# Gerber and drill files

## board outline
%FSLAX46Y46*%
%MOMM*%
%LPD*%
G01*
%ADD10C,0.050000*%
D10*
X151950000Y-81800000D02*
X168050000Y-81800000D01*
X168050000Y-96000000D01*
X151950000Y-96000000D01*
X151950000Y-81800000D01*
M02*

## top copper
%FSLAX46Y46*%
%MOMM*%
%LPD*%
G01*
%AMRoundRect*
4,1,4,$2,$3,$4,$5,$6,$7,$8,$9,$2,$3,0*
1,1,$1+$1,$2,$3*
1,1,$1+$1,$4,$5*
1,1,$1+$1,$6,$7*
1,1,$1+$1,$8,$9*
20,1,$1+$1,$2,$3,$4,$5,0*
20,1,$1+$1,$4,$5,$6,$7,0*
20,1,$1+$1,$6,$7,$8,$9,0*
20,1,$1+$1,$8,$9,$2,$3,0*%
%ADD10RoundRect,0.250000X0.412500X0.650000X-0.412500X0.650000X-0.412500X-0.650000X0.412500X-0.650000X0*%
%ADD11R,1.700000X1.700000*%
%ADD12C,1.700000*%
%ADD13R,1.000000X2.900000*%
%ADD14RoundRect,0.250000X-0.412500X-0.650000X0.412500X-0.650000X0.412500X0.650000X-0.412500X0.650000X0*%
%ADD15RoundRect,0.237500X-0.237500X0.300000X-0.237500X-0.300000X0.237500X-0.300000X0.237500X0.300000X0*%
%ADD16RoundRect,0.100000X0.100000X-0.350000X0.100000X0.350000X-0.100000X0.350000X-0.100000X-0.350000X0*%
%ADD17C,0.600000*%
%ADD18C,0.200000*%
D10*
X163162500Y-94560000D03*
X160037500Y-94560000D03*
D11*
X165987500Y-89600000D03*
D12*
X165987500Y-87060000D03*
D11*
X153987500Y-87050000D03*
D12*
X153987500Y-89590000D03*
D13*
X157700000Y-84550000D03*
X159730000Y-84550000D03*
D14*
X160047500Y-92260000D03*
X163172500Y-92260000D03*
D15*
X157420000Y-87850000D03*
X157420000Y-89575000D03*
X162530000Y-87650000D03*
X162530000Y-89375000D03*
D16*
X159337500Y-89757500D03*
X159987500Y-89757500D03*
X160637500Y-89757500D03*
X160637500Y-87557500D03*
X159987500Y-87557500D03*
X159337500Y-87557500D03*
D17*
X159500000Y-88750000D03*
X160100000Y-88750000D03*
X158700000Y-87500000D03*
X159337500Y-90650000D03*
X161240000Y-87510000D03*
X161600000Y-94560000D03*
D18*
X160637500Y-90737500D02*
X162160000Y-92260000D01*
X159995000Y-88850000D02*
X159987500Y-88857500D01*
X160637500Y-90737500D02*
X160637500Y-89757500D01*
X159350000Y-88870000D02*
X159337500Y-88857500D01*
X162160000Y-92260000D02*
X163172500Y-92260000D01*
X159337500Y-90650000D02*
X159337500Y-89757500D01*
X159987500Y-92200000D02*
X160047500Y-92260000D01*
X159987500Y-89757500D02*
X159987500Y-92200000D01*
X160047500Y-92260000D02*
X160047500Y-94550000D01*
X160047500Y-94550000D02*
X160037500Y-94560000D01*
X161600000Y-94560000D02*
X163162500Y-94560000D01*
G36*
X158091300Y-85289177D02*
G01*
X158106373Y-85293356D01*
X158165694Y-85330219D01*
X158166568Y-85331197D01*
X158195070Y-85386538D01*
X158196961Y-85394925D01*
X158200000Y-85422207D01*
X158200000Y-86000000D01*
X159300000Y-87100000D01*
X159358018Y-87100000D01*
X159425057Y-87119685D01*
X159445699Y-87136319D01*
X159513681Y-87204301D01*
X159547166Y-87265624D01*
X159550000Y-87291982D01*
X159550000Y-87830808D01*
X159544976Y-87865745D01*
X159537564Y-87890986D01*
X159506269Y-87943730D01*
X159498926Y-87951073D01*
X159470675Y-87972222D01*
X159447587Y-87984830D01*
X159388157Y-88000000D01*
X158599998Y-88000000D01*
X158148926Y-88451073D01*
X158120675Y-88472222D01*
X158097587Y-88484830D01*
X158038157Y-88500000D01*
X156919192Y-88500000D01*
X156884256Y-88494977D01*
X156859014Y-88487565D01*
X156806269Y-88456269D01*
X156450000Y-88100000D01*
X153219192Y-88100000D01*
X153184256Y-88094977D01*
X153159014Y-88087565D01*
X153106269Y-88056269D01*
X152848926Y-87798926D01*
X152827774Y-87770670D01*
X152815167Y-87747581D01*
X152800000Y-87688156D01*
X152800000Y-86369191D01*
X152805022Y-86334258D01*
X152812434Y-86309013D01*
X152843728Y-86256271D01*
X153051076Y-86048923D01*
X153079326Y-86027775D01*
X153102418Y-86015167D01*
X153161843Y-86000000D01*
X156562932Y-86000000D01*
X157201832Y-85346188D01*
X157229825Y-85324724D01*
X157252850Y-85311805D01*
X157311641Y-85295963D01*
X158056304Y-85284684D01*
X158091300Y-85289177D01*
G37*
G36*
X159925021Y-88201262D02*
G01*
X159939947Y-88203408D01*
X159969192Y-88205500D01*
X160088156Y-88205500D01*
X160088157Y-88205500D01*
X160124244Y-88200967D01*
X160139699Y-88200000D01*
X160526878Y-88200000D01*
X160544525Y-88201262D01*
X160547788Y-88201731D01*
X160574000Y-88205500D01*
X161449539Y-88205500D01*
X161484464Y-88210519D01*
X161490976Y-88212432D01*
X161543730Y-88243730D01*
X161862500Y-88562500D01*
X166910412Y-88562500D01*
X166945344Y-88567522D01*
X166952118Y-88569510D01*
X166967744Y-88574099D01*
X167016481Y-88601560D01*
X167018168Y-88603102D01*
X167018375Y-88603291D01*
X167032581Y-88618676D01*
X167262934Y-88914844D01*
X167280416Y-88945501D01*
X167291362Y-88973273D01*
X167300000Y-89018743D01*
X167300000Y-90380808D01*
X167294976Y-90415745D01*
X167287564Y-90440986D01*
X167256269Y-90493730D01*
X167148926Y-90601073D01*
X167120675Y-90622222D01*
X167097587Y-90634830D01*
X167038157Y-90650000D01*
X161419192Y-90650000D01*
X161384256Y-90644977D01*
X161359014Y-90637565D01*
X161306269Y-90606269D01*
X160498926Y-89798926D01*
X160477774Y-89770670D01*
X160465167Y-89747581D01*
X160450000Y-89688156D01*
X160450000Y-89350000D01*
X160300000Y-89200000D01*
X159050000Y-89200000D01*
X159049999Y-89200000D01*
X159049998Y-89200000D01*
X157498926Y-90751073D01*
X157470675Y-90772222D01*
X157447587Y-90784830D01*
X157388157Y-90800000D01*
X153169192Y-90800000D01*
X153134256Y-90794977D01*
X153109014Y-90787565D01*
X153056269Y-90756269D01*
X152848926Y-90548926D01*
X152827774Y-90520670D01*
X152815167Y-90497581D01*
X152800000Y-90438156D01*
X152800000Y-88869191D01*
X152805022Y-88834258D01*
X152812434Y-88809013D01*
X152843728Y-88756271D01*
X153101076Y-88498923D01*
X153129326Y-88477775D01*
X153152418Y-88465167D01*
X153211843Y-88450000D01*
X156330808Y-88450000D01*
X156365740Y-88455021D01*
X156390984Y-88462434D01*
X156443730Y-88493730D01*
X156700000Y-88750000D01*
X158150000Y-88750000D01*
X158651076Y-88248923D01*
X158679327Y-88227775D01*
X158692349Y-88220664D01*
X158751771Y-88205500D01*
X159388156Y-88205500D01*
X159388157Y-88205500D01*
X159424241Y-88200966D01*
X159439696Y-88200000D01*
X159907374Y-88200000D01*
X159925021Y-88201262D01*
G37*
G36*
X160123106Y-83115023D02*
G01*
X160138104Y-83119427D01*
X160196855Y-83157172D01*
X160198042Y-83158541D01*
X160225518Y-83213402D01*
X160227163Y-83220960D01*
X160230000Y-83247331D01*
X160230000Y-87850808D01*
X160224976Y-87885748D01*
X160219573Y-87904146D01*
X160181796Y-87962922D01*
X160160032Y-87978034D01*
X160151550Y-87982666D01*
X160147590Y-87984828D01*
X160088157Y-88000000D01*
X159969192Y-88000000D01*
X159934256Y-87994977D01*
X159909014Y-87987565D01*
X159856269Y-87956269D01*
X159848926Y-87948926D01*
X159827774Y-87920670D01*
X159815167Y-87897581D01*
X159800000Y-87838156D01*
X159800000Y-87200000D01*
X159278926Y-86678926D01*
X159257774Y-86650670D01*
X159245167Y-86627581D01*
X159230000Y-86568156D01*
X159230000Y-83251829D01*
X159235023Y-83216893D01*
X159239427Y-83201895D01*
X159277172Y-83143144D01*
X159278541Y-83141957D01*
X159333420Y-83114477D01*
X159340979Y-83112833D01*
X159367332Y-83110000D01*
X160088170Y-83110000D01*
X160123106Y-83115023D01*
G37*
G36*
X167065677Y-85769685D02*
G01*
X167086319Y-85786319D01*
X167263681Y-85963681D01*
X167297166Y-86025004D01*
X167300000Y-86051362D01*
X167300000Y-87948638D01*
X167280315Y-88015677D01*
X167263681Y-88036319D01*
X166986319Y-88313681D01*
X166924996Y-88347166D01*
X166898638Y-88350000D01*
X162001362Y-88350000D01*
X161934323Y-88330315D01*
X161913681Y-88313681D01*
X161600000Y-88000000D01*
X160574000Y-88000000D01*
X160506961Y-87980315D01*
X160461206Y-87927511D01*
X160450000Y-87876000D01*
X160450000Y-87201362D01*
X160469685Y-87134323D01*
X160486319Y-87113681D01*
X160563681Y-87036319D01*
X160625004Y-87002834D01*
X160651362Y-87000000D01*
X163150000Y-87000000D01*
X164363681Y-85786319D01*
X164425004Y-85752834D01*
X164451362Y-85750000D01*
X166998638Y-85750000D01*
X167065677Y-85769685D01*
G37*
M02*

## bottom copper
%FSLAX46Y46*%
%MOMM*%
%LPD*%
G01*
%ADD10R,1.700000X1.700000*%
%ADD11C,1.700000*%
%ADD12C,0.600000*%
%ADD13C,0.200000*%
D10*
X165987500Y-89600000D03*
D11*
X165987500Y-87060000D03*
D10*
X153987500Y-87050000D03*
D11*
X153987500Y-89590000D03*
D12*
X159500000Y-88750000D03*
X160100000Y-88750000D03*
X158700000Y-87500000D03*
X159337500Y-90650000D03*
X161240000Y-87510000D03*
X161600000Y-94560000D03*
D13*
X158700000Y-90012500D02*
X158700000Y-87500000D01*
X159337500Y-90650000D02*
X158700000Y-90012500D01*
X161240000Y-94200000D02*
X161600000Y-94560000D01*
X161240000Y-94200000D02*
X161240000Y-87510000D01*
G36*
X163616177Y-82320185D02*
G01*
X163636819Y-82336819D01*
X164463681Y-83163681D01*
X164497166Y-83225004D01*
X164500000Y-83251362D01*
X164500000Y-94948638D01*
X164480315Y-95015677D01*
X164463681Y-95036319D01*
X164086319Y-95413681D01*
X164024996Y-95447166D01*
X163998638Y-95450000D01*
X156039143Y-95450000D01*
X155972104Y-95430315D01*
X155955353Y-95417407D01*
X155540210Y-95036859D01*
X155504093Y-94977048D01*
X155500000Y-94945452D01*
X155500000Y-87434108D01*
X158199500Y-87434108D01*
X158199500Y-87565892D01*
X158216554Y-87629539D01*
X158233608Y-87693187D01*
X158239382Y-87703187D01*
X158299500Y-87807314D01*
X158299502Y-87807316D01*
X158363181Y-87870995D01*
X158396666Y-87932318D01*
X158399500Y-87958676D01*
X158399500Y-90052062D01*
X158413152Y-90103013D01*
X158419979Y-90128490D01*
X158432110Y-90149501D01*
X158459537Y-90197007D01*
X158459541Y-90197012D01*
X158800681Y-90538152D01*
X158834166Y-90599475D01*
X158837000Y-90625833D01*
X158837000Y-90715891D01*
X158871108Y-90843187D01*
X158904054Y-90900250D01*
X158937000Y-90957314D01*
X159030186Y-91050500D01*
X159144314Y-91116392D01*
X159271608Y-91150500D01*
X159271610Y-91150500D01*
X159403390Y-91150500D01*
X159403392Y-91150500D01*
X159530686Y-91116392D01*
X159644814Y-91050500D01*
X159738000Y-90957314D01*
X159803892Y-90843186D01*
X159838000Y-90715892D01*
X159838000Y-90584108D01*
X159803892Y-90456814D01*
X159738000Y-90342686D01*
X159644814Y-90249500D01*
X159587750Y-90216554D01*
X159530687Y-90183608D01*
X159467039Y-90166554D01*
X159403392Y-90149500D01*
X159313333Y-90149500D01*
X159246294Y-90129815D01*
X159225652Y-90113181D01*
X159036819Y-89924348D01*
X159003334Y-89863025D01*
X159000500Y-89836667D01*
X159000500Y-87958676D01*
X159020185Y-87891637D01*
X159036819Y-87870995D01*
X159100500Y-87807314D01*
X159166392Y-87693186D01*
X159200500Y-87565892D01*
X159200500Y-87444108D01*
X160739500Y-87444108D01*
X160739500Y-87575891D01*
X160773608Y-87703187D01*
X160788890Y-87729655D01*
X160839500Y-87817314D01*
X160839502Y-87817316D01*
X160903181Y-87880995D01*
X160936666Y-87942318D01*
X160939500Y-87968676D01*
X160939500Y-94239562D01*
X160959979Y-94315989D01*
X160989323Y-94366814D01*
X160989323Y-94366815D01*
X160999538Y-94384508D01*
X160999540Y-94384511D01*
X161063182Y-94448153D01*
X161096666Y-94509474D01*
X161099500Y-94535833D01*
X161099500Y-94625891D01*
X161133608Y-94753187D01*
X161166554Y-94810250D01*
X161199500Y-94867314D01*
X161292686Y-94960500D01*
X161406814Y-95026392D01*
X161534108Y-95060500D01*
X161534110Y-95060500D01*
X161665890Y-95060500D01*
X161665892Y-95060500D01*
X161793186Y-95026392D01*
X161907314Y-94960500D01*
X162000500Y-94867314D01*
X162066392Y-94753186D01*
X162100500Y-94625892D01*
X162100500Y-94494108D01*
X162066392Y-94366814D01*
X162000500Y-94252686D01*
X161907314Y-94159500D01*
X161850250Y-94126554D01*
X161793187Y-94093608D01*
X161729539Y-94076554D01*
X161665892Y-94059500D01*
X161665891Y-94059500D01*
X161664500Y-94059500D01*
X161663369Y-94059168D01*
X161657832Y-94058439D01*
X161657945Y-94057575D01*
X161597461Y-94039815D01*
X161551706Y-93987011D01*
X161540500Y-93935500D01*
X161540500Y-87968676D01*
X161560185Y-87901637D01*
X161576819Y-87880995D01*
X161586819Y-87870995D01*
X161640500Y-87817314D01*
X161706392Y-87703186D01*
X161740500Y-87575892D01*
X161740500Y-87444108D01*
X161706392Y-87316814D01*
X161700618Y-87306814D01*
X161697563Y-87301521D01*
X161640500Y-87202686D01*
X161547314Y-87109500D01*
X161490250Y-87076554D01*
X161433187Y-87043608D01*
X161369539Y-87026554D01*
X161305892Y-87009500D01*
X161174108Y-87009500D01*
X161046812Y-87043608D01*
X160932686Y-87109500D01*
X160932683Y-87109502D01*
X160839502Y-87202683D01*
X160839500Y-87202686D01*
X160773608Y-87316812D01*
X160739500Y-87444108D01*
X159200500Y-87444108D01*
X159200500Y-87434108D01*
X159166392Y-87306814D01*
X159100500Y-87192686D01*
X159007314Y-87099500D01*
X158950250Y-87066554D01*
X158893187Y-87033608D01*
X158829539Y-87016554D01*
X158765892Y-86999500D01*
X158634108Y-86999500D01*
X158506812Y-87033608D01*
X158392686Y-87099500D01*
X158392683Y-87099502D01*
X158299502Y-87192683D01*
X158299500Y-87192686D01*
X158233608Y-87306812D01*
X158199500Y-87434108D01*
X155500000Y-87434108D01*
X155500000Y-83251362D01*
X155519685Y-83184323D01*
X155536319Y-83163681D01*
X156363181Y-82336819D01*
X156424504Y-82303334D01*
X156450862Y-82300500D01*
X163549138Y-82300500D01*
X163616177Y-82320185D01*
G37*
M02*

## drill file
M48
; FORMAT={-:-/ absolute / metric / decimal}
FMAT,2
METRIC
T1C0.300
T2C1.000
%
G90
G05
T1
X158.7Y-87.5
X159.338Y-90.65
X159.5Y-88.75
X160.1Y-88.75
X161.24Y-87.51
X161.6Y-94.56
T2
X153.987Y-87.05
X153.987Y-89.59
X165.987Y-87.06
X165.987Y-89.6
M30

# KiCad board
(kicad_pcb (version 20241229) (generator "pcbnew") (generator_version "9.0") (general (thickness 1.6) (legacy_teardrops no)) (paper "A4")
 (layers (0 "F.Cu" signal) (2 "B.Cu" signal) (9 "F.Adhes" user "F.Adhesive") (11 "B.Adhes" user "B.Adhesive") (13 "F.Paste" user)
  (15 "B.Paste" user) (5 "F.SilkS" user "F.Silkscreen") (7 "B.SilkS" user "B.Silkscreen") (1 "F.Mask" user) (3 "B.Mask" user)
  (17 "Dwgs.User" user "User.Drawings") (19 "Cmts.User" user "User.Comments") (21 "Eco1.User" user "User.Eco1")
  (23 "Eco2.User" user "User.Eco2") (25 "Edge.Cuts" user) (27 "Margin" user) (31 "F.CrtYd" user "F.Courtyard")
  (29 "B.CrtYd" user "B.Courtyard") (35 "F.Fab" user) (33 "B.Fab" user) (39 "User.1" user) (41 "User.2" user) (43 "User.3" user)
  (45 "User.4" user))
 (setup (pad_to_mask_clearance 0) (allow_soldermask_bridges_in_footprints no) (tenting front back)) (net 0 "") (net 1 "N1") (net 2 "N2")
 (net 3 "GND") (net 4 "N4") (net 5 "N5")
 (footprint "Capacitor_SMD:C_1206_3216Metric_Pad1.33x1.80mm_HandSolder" (layer "F.Cu") (at 161.6 94.56 180)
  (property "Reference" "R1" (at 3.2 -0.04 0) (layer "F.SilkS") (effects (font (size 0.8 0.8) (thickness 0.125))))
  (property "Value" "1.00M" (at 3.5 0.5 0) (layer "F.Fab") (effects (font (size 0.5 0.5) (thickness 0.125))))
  (pad "1" smd roundrect (at -1.5625 0 180) (size 1.325 1.8) (layers "F.Cu" "F.Mask" "F.Paste") (roundrect_rratio 0.188679) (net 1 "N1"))
  (pad "2" smd roundrect (at 1.5625 0 180) (size 1.325 1.8) (layers "F.Cu" "F.Mask" "F.Paste") (roundrect_rratio 0.188679) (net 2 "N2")))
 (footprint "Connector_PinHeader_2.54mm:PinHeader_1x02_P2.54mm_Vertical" (layer "F.Cu") (at 165.9875 89.6 180)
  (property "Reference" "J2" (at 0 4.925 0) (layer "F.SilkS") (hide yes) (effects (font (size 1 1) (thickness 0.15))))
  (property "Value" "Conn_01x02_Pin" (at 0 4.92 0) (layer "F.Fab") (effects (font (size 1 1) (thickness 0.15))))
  (pad "1" thru_hole rect (at 0 0 180) (size 1.7 1.7) (drill 1) (layers "*.Cu" "*.Mask") (remove_unused_layers no) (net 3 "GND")
   (zone_connect 2))
  (pad "2" thru_hole circle (at 0 2.54 180) (size 1.7 1.7) (drill 1) (layers "*.Cu" "*.Mask") (remove_unused_layers no) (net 1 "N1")
   (zone_connect 2)))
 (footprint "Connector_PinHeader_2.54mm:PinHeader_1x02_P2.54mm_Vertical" (layer "F.Cu") (at 153.9875 87.05)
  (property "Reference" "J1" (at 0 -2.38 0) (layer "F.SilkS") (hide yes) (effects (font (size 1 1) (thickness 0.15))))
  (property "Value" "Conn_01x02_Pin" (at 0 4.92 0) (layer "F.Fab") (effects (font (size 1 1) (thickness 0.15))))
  (pad "1" thru_hole rect (at 0 0) (size 1.7 1.7) (drill 1) (layers "*.Cu" "*.Mask") (remove_unused_layers no) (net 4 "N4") (clearance 0.1)
   (zone_connect 2))
  (pad "2" thru_hole circle (at 0 2.54) (size 1.7 1.7) (drill 1) (layers "*.Cu" "*.Mask") (remove_unused_layers no) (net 3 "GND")
   (zone_connect 2)))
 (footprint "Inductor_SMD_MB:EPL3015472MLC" (layer "F.Cu") (at 158.715 84.55)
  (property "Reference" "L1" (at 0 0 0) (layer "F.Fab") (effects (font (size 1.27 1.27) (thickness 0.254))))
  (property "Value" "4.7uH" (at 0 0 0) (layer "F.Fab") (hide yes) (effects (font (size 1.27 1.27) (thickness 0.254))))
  (pad "1" smd rect (at -1.015 0) (size 1 2.9) (layers "F.Cu" "F.Mask" "F.Paste") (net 4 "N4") (zone_connect 2))
  (pad "2" smd rect (at 1.015 0) (size 1 2.9) (layers "F.Cu" "F.Mask" "F.Paste") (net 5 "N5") (zone_connect 2)))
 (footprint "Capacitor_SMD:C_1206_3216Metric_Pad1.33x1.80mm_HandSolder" (layer "F.Cu") (at 161.61 92.26)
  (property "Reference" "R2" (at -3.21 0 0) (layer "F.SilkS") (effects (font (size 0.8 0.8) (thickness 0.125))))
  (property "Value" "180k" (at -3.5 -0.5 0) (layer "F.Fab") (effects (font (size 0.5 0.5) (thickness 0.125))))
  (pad "1" smd roundrect (at -1.5625 0) (size 1.325 1.8) (layers "F.Cu" "F.Mask" "F.Paste") (roundrect_rratio 0.188679) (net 2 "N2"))
  (pad "2" smd roundrect (at 1.5625 0) (size 1.325 1.8) (layers "F.Cu" "F.Mask" "F.Paste") (roundrect_rratio 0.188679) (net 3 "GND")
   (zone_connect 2)))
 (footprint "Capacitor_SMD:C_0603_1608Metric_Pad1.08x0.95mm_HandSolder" (layer "F.Cu") (at 157.42 88.7125 -90)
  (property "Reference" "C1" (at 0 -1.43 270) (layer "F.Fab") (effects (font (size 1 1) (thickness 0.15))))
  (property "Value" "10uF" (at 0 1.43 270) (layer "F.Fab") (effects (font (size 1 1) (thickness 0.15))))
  (pad "1" smd roundrect (at -0.8625 0 270) (size 1.075 0.95) (layers "F.Cu" "F.Mask" "F.Paste") (roundrect_rratio 0.25) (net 4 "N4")
   (clearance 0.1) (zone_connect 2))
  (pad "2" smd roundrect (at 0.8625 0 270) (size 1.075 0.95) (layers "F.Cu" "F.Mask" "F.Paste") (roundrect_rratio 0.25) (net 3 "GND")
   (clearance 0.1) (zone_connect 2)))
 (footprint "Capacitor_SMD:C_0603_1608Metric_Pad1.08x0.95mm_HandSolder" (layer "F.Cu") (at 162.53 88.5125 -90)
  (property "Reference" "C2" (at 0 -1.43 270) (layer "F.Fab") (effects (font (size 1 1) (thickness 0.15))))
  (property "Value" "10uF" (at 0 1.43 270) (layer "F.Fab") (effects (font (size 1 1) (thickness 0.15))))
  (pad "1" smd roundrect (at -0.8625 0 270) (size 1.075 0.95) (layers "F.Cu" "F.Mask" "F.Paste") (roundrect_rratio 0.25) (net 1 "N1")
   (clearance 0.1) (zone_connect 2))
  (pad "2" smd roundrect (at 0.8625 0 270) (size 1.075 0.95) (layers "F.Cu" "F.Mask" "F.Paste") (roundrect_rratio 0.25) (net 3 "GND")
   (clearance 0.1) (zone_connect 2)))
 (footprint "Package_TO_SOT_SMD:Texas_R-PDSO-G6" (layer "F.Cu") (at 159.9875 88.6575 90)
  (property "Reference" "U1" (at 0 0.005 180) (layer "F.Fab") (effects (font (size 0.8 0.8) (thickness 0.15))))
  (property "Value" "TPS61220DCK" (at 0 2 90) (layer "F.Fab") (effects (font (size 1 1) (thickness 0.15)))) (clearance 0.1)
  (pad "1" smd roundrect (at -1.1 -0.65 90) (size 0.9 0.4) (layers "F.Cu" "F.Mask" "F.Paste") (roundrect_rratio 0.25) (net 4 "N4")
   (clearance 0.1))
  (pad "2" smd roundrect (at -1.1 0 90) (size 0.9 0.4) (layers "F.Cu" "F.Mask" "F.Paste") (roundrect_rratio 0.25) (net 2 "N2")
   (clearance 0.1))
  (pad "3" smd roundrect (at -1.1 0.65 90) (size 0.9 0.4) (layers "F.Cu" "F.Mask" "F.Paste") (roundrect_rratio 0.25) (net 3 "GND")
   (zone_connect 2))
  (pad "4" smd roundrect (at 1.1 0.65 90) (size 0.9 0.4) (layers "F.Cu" "F.Mask" "F.Paste") (roundrect_rratio 0.25) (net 1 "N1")
   (clearance 0.1) (zone_connect 2))
  (pad "5" smd roundrect (at 1.1 0 90) (size 0.9 0.4) (layers "F.Cu" "F.Mask" "F.Paste") (roundrect_rratio 0.25) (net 5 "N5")
   (clearance 0.1) (zone_connect 2))
  (pad "6" smd roundrect (at 1.1 -0.65 90) (size 0.9 0.4) (layers "F.Cu" "F.Mask" "F.Paste") (roundrect_rratio 0.25) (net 4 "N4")
   (clearance 0.1) (zone_connect 2)))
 (gr_rect (start 151.95 81.8) (end 168.05 96) (stroke (width 0.05) (type solid)) (fill no) (layer "Edge.Cuts"))
 (segment (start 160.6375 90.7375) (end 162.16 92.26) (width 0.2) (layer "F.Cu") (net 3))
 (segment (start 159.995 88.85) (end 159.9875 88.8575) (width 0.2) (layer "F.Cu") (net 3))
 (segment (start 160.6375 90.7375) (end 160.6375 89.7575) (width 0.2) (layer "F.Cu") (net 3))
 (segment (start 159.35 88.87) (end 159.3375 88.8575) (width 0.2) (layer "F.Cu") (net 3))
 (segment (start 162.16 92.26) (end 163.1725 92.26) (width 0.2) (layer "F.Cu") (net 3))
 (via (at 159.5 88.75) (size 0.6) (drill 0.3) (layers "F.Cu" "B.Cu") (free yes) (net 3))
 (via (at 160.1 88.75) (size 0.6) (drill 0.3) (layers "F.Cu" "B.Cu") (free yes) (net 3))
 (segment (start 159.3375 90.65) (end 159.3375 89.7575) (width 0.2) (layer "F.Cu") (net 4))
 (via (at 158.7 87.5) (size 0.6) (drill 0.3) (layers "F.Cu" "B.Cu") (free yes) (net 4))
 (via (at 159.3375 90.65) (size 0.6) (drill 0.3) (layers "F.Cu" "B.Cu") (free yes) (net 4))
 (segment (start 158.7 90.0125) (end 158.7 87.5) (width 0.2) (layer "B.Cu") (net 4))
 (segment (start 159.3375 90.65) (end 158.7 90.0125) (width 0.2) (layer "B.Cu") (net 4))
 (segment (start 159.9875 92.2) (end 160.0475 92.26) (width 0.2) (layer "F.Cu") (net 2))
 (segment (start 159.9875 89.7575) (end 159.9875 92.2) (width 0.2) (layer "F.Cu") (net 2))
 (segment (start 160.0475 92.26) (end 160.0475 94.55) (width 0.2) (layer "F.Cu") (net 2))
 (segment (start 160.0475 94.55) (end 160.0375 94.56) (width 0.2) (layer "F.Cu") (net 2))
 (segment (start 161.6 94.56) (end 163.1625 94.56) (width 0.2) (layer "F.Cu") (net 1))
 (via (at 161.24 87.51) (size 0.6) (drill 0.3) (layers "F.Cu" "B.Cu") (free yes) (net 1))
 (via (at 161.6 94.56) (size 0.6) (drill 0.3) (layers "F.Cu" "B.Cu") (free yes) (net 1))
 (segment (start 161.24 94.2) (end 161.6 94.56) (width 0.2) (layer "B.Cu") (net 1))
 (segment (start 161.24 94.2) (end 161.24 87.51) (width 0.2) (layer "B.Cu") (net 1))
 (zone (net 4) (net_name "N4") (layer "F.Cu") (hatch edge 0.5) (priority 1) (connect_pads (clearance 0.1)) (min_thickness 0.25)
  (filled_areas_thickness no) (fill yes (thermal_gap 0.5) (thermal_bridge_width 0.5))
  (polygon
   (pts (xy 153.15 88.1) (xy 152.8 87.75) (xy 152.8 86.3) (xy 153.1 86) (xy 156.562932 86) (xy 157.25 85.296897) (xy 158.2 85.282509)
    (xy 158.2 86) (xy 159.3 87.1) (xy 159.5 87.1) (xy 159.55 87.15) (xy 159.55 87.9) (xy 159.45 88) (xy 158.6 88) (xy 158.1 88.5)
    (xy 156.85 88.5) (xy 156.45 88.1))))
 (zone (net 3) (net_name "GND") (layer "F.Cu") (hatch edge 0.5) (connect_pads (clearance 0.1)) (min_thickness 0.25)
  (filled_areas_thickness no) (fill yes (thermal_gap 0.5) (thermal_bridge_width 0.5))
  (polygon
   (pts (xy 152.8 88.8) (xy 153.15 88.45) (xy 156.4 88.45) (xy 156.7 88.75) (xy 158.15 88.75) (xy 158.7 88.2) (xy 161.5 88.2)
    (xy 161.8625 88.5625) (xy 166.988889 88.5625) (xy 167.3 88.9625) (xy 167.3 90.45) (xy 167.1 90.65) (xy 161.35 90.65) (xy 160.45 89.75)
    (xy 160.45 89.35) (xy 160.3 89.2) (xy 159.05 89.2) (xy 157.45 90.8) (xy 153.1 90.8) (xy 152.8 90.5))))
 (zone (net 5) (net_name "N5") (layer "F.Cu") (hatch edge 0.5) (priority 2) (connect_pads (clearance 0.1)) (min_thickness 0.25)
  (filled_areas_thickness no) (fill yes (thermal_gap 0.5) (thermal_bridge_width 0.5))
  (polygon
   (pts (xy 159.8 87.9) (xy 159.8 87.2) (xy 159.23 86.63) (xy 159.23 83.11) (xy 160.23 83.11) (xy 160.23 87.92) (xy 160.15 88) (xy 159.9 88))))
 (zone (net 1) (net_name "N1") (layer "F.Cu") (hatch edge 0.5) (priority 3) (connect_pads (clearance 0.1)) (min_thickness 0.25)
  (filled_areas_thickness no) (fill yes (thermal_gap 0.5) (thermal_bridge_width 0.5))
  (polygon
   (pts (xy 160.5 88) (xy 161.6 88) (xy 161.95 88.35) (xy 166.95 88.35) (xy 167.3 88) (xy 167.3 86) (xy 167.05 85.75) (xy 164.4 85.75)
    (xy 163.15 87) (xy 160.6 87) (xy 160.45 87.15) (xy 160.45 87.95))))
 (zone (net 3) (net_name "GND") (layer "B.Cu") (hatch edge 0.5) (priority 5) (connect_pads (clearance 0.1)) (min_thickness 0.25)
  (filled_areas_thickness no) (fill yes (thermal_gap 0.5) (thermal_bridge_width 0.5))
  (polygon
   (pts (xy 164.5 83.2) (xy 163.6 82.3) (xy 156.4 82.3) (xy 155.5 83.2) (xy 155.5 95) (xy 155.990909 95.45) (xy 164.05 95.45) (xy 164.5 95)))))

